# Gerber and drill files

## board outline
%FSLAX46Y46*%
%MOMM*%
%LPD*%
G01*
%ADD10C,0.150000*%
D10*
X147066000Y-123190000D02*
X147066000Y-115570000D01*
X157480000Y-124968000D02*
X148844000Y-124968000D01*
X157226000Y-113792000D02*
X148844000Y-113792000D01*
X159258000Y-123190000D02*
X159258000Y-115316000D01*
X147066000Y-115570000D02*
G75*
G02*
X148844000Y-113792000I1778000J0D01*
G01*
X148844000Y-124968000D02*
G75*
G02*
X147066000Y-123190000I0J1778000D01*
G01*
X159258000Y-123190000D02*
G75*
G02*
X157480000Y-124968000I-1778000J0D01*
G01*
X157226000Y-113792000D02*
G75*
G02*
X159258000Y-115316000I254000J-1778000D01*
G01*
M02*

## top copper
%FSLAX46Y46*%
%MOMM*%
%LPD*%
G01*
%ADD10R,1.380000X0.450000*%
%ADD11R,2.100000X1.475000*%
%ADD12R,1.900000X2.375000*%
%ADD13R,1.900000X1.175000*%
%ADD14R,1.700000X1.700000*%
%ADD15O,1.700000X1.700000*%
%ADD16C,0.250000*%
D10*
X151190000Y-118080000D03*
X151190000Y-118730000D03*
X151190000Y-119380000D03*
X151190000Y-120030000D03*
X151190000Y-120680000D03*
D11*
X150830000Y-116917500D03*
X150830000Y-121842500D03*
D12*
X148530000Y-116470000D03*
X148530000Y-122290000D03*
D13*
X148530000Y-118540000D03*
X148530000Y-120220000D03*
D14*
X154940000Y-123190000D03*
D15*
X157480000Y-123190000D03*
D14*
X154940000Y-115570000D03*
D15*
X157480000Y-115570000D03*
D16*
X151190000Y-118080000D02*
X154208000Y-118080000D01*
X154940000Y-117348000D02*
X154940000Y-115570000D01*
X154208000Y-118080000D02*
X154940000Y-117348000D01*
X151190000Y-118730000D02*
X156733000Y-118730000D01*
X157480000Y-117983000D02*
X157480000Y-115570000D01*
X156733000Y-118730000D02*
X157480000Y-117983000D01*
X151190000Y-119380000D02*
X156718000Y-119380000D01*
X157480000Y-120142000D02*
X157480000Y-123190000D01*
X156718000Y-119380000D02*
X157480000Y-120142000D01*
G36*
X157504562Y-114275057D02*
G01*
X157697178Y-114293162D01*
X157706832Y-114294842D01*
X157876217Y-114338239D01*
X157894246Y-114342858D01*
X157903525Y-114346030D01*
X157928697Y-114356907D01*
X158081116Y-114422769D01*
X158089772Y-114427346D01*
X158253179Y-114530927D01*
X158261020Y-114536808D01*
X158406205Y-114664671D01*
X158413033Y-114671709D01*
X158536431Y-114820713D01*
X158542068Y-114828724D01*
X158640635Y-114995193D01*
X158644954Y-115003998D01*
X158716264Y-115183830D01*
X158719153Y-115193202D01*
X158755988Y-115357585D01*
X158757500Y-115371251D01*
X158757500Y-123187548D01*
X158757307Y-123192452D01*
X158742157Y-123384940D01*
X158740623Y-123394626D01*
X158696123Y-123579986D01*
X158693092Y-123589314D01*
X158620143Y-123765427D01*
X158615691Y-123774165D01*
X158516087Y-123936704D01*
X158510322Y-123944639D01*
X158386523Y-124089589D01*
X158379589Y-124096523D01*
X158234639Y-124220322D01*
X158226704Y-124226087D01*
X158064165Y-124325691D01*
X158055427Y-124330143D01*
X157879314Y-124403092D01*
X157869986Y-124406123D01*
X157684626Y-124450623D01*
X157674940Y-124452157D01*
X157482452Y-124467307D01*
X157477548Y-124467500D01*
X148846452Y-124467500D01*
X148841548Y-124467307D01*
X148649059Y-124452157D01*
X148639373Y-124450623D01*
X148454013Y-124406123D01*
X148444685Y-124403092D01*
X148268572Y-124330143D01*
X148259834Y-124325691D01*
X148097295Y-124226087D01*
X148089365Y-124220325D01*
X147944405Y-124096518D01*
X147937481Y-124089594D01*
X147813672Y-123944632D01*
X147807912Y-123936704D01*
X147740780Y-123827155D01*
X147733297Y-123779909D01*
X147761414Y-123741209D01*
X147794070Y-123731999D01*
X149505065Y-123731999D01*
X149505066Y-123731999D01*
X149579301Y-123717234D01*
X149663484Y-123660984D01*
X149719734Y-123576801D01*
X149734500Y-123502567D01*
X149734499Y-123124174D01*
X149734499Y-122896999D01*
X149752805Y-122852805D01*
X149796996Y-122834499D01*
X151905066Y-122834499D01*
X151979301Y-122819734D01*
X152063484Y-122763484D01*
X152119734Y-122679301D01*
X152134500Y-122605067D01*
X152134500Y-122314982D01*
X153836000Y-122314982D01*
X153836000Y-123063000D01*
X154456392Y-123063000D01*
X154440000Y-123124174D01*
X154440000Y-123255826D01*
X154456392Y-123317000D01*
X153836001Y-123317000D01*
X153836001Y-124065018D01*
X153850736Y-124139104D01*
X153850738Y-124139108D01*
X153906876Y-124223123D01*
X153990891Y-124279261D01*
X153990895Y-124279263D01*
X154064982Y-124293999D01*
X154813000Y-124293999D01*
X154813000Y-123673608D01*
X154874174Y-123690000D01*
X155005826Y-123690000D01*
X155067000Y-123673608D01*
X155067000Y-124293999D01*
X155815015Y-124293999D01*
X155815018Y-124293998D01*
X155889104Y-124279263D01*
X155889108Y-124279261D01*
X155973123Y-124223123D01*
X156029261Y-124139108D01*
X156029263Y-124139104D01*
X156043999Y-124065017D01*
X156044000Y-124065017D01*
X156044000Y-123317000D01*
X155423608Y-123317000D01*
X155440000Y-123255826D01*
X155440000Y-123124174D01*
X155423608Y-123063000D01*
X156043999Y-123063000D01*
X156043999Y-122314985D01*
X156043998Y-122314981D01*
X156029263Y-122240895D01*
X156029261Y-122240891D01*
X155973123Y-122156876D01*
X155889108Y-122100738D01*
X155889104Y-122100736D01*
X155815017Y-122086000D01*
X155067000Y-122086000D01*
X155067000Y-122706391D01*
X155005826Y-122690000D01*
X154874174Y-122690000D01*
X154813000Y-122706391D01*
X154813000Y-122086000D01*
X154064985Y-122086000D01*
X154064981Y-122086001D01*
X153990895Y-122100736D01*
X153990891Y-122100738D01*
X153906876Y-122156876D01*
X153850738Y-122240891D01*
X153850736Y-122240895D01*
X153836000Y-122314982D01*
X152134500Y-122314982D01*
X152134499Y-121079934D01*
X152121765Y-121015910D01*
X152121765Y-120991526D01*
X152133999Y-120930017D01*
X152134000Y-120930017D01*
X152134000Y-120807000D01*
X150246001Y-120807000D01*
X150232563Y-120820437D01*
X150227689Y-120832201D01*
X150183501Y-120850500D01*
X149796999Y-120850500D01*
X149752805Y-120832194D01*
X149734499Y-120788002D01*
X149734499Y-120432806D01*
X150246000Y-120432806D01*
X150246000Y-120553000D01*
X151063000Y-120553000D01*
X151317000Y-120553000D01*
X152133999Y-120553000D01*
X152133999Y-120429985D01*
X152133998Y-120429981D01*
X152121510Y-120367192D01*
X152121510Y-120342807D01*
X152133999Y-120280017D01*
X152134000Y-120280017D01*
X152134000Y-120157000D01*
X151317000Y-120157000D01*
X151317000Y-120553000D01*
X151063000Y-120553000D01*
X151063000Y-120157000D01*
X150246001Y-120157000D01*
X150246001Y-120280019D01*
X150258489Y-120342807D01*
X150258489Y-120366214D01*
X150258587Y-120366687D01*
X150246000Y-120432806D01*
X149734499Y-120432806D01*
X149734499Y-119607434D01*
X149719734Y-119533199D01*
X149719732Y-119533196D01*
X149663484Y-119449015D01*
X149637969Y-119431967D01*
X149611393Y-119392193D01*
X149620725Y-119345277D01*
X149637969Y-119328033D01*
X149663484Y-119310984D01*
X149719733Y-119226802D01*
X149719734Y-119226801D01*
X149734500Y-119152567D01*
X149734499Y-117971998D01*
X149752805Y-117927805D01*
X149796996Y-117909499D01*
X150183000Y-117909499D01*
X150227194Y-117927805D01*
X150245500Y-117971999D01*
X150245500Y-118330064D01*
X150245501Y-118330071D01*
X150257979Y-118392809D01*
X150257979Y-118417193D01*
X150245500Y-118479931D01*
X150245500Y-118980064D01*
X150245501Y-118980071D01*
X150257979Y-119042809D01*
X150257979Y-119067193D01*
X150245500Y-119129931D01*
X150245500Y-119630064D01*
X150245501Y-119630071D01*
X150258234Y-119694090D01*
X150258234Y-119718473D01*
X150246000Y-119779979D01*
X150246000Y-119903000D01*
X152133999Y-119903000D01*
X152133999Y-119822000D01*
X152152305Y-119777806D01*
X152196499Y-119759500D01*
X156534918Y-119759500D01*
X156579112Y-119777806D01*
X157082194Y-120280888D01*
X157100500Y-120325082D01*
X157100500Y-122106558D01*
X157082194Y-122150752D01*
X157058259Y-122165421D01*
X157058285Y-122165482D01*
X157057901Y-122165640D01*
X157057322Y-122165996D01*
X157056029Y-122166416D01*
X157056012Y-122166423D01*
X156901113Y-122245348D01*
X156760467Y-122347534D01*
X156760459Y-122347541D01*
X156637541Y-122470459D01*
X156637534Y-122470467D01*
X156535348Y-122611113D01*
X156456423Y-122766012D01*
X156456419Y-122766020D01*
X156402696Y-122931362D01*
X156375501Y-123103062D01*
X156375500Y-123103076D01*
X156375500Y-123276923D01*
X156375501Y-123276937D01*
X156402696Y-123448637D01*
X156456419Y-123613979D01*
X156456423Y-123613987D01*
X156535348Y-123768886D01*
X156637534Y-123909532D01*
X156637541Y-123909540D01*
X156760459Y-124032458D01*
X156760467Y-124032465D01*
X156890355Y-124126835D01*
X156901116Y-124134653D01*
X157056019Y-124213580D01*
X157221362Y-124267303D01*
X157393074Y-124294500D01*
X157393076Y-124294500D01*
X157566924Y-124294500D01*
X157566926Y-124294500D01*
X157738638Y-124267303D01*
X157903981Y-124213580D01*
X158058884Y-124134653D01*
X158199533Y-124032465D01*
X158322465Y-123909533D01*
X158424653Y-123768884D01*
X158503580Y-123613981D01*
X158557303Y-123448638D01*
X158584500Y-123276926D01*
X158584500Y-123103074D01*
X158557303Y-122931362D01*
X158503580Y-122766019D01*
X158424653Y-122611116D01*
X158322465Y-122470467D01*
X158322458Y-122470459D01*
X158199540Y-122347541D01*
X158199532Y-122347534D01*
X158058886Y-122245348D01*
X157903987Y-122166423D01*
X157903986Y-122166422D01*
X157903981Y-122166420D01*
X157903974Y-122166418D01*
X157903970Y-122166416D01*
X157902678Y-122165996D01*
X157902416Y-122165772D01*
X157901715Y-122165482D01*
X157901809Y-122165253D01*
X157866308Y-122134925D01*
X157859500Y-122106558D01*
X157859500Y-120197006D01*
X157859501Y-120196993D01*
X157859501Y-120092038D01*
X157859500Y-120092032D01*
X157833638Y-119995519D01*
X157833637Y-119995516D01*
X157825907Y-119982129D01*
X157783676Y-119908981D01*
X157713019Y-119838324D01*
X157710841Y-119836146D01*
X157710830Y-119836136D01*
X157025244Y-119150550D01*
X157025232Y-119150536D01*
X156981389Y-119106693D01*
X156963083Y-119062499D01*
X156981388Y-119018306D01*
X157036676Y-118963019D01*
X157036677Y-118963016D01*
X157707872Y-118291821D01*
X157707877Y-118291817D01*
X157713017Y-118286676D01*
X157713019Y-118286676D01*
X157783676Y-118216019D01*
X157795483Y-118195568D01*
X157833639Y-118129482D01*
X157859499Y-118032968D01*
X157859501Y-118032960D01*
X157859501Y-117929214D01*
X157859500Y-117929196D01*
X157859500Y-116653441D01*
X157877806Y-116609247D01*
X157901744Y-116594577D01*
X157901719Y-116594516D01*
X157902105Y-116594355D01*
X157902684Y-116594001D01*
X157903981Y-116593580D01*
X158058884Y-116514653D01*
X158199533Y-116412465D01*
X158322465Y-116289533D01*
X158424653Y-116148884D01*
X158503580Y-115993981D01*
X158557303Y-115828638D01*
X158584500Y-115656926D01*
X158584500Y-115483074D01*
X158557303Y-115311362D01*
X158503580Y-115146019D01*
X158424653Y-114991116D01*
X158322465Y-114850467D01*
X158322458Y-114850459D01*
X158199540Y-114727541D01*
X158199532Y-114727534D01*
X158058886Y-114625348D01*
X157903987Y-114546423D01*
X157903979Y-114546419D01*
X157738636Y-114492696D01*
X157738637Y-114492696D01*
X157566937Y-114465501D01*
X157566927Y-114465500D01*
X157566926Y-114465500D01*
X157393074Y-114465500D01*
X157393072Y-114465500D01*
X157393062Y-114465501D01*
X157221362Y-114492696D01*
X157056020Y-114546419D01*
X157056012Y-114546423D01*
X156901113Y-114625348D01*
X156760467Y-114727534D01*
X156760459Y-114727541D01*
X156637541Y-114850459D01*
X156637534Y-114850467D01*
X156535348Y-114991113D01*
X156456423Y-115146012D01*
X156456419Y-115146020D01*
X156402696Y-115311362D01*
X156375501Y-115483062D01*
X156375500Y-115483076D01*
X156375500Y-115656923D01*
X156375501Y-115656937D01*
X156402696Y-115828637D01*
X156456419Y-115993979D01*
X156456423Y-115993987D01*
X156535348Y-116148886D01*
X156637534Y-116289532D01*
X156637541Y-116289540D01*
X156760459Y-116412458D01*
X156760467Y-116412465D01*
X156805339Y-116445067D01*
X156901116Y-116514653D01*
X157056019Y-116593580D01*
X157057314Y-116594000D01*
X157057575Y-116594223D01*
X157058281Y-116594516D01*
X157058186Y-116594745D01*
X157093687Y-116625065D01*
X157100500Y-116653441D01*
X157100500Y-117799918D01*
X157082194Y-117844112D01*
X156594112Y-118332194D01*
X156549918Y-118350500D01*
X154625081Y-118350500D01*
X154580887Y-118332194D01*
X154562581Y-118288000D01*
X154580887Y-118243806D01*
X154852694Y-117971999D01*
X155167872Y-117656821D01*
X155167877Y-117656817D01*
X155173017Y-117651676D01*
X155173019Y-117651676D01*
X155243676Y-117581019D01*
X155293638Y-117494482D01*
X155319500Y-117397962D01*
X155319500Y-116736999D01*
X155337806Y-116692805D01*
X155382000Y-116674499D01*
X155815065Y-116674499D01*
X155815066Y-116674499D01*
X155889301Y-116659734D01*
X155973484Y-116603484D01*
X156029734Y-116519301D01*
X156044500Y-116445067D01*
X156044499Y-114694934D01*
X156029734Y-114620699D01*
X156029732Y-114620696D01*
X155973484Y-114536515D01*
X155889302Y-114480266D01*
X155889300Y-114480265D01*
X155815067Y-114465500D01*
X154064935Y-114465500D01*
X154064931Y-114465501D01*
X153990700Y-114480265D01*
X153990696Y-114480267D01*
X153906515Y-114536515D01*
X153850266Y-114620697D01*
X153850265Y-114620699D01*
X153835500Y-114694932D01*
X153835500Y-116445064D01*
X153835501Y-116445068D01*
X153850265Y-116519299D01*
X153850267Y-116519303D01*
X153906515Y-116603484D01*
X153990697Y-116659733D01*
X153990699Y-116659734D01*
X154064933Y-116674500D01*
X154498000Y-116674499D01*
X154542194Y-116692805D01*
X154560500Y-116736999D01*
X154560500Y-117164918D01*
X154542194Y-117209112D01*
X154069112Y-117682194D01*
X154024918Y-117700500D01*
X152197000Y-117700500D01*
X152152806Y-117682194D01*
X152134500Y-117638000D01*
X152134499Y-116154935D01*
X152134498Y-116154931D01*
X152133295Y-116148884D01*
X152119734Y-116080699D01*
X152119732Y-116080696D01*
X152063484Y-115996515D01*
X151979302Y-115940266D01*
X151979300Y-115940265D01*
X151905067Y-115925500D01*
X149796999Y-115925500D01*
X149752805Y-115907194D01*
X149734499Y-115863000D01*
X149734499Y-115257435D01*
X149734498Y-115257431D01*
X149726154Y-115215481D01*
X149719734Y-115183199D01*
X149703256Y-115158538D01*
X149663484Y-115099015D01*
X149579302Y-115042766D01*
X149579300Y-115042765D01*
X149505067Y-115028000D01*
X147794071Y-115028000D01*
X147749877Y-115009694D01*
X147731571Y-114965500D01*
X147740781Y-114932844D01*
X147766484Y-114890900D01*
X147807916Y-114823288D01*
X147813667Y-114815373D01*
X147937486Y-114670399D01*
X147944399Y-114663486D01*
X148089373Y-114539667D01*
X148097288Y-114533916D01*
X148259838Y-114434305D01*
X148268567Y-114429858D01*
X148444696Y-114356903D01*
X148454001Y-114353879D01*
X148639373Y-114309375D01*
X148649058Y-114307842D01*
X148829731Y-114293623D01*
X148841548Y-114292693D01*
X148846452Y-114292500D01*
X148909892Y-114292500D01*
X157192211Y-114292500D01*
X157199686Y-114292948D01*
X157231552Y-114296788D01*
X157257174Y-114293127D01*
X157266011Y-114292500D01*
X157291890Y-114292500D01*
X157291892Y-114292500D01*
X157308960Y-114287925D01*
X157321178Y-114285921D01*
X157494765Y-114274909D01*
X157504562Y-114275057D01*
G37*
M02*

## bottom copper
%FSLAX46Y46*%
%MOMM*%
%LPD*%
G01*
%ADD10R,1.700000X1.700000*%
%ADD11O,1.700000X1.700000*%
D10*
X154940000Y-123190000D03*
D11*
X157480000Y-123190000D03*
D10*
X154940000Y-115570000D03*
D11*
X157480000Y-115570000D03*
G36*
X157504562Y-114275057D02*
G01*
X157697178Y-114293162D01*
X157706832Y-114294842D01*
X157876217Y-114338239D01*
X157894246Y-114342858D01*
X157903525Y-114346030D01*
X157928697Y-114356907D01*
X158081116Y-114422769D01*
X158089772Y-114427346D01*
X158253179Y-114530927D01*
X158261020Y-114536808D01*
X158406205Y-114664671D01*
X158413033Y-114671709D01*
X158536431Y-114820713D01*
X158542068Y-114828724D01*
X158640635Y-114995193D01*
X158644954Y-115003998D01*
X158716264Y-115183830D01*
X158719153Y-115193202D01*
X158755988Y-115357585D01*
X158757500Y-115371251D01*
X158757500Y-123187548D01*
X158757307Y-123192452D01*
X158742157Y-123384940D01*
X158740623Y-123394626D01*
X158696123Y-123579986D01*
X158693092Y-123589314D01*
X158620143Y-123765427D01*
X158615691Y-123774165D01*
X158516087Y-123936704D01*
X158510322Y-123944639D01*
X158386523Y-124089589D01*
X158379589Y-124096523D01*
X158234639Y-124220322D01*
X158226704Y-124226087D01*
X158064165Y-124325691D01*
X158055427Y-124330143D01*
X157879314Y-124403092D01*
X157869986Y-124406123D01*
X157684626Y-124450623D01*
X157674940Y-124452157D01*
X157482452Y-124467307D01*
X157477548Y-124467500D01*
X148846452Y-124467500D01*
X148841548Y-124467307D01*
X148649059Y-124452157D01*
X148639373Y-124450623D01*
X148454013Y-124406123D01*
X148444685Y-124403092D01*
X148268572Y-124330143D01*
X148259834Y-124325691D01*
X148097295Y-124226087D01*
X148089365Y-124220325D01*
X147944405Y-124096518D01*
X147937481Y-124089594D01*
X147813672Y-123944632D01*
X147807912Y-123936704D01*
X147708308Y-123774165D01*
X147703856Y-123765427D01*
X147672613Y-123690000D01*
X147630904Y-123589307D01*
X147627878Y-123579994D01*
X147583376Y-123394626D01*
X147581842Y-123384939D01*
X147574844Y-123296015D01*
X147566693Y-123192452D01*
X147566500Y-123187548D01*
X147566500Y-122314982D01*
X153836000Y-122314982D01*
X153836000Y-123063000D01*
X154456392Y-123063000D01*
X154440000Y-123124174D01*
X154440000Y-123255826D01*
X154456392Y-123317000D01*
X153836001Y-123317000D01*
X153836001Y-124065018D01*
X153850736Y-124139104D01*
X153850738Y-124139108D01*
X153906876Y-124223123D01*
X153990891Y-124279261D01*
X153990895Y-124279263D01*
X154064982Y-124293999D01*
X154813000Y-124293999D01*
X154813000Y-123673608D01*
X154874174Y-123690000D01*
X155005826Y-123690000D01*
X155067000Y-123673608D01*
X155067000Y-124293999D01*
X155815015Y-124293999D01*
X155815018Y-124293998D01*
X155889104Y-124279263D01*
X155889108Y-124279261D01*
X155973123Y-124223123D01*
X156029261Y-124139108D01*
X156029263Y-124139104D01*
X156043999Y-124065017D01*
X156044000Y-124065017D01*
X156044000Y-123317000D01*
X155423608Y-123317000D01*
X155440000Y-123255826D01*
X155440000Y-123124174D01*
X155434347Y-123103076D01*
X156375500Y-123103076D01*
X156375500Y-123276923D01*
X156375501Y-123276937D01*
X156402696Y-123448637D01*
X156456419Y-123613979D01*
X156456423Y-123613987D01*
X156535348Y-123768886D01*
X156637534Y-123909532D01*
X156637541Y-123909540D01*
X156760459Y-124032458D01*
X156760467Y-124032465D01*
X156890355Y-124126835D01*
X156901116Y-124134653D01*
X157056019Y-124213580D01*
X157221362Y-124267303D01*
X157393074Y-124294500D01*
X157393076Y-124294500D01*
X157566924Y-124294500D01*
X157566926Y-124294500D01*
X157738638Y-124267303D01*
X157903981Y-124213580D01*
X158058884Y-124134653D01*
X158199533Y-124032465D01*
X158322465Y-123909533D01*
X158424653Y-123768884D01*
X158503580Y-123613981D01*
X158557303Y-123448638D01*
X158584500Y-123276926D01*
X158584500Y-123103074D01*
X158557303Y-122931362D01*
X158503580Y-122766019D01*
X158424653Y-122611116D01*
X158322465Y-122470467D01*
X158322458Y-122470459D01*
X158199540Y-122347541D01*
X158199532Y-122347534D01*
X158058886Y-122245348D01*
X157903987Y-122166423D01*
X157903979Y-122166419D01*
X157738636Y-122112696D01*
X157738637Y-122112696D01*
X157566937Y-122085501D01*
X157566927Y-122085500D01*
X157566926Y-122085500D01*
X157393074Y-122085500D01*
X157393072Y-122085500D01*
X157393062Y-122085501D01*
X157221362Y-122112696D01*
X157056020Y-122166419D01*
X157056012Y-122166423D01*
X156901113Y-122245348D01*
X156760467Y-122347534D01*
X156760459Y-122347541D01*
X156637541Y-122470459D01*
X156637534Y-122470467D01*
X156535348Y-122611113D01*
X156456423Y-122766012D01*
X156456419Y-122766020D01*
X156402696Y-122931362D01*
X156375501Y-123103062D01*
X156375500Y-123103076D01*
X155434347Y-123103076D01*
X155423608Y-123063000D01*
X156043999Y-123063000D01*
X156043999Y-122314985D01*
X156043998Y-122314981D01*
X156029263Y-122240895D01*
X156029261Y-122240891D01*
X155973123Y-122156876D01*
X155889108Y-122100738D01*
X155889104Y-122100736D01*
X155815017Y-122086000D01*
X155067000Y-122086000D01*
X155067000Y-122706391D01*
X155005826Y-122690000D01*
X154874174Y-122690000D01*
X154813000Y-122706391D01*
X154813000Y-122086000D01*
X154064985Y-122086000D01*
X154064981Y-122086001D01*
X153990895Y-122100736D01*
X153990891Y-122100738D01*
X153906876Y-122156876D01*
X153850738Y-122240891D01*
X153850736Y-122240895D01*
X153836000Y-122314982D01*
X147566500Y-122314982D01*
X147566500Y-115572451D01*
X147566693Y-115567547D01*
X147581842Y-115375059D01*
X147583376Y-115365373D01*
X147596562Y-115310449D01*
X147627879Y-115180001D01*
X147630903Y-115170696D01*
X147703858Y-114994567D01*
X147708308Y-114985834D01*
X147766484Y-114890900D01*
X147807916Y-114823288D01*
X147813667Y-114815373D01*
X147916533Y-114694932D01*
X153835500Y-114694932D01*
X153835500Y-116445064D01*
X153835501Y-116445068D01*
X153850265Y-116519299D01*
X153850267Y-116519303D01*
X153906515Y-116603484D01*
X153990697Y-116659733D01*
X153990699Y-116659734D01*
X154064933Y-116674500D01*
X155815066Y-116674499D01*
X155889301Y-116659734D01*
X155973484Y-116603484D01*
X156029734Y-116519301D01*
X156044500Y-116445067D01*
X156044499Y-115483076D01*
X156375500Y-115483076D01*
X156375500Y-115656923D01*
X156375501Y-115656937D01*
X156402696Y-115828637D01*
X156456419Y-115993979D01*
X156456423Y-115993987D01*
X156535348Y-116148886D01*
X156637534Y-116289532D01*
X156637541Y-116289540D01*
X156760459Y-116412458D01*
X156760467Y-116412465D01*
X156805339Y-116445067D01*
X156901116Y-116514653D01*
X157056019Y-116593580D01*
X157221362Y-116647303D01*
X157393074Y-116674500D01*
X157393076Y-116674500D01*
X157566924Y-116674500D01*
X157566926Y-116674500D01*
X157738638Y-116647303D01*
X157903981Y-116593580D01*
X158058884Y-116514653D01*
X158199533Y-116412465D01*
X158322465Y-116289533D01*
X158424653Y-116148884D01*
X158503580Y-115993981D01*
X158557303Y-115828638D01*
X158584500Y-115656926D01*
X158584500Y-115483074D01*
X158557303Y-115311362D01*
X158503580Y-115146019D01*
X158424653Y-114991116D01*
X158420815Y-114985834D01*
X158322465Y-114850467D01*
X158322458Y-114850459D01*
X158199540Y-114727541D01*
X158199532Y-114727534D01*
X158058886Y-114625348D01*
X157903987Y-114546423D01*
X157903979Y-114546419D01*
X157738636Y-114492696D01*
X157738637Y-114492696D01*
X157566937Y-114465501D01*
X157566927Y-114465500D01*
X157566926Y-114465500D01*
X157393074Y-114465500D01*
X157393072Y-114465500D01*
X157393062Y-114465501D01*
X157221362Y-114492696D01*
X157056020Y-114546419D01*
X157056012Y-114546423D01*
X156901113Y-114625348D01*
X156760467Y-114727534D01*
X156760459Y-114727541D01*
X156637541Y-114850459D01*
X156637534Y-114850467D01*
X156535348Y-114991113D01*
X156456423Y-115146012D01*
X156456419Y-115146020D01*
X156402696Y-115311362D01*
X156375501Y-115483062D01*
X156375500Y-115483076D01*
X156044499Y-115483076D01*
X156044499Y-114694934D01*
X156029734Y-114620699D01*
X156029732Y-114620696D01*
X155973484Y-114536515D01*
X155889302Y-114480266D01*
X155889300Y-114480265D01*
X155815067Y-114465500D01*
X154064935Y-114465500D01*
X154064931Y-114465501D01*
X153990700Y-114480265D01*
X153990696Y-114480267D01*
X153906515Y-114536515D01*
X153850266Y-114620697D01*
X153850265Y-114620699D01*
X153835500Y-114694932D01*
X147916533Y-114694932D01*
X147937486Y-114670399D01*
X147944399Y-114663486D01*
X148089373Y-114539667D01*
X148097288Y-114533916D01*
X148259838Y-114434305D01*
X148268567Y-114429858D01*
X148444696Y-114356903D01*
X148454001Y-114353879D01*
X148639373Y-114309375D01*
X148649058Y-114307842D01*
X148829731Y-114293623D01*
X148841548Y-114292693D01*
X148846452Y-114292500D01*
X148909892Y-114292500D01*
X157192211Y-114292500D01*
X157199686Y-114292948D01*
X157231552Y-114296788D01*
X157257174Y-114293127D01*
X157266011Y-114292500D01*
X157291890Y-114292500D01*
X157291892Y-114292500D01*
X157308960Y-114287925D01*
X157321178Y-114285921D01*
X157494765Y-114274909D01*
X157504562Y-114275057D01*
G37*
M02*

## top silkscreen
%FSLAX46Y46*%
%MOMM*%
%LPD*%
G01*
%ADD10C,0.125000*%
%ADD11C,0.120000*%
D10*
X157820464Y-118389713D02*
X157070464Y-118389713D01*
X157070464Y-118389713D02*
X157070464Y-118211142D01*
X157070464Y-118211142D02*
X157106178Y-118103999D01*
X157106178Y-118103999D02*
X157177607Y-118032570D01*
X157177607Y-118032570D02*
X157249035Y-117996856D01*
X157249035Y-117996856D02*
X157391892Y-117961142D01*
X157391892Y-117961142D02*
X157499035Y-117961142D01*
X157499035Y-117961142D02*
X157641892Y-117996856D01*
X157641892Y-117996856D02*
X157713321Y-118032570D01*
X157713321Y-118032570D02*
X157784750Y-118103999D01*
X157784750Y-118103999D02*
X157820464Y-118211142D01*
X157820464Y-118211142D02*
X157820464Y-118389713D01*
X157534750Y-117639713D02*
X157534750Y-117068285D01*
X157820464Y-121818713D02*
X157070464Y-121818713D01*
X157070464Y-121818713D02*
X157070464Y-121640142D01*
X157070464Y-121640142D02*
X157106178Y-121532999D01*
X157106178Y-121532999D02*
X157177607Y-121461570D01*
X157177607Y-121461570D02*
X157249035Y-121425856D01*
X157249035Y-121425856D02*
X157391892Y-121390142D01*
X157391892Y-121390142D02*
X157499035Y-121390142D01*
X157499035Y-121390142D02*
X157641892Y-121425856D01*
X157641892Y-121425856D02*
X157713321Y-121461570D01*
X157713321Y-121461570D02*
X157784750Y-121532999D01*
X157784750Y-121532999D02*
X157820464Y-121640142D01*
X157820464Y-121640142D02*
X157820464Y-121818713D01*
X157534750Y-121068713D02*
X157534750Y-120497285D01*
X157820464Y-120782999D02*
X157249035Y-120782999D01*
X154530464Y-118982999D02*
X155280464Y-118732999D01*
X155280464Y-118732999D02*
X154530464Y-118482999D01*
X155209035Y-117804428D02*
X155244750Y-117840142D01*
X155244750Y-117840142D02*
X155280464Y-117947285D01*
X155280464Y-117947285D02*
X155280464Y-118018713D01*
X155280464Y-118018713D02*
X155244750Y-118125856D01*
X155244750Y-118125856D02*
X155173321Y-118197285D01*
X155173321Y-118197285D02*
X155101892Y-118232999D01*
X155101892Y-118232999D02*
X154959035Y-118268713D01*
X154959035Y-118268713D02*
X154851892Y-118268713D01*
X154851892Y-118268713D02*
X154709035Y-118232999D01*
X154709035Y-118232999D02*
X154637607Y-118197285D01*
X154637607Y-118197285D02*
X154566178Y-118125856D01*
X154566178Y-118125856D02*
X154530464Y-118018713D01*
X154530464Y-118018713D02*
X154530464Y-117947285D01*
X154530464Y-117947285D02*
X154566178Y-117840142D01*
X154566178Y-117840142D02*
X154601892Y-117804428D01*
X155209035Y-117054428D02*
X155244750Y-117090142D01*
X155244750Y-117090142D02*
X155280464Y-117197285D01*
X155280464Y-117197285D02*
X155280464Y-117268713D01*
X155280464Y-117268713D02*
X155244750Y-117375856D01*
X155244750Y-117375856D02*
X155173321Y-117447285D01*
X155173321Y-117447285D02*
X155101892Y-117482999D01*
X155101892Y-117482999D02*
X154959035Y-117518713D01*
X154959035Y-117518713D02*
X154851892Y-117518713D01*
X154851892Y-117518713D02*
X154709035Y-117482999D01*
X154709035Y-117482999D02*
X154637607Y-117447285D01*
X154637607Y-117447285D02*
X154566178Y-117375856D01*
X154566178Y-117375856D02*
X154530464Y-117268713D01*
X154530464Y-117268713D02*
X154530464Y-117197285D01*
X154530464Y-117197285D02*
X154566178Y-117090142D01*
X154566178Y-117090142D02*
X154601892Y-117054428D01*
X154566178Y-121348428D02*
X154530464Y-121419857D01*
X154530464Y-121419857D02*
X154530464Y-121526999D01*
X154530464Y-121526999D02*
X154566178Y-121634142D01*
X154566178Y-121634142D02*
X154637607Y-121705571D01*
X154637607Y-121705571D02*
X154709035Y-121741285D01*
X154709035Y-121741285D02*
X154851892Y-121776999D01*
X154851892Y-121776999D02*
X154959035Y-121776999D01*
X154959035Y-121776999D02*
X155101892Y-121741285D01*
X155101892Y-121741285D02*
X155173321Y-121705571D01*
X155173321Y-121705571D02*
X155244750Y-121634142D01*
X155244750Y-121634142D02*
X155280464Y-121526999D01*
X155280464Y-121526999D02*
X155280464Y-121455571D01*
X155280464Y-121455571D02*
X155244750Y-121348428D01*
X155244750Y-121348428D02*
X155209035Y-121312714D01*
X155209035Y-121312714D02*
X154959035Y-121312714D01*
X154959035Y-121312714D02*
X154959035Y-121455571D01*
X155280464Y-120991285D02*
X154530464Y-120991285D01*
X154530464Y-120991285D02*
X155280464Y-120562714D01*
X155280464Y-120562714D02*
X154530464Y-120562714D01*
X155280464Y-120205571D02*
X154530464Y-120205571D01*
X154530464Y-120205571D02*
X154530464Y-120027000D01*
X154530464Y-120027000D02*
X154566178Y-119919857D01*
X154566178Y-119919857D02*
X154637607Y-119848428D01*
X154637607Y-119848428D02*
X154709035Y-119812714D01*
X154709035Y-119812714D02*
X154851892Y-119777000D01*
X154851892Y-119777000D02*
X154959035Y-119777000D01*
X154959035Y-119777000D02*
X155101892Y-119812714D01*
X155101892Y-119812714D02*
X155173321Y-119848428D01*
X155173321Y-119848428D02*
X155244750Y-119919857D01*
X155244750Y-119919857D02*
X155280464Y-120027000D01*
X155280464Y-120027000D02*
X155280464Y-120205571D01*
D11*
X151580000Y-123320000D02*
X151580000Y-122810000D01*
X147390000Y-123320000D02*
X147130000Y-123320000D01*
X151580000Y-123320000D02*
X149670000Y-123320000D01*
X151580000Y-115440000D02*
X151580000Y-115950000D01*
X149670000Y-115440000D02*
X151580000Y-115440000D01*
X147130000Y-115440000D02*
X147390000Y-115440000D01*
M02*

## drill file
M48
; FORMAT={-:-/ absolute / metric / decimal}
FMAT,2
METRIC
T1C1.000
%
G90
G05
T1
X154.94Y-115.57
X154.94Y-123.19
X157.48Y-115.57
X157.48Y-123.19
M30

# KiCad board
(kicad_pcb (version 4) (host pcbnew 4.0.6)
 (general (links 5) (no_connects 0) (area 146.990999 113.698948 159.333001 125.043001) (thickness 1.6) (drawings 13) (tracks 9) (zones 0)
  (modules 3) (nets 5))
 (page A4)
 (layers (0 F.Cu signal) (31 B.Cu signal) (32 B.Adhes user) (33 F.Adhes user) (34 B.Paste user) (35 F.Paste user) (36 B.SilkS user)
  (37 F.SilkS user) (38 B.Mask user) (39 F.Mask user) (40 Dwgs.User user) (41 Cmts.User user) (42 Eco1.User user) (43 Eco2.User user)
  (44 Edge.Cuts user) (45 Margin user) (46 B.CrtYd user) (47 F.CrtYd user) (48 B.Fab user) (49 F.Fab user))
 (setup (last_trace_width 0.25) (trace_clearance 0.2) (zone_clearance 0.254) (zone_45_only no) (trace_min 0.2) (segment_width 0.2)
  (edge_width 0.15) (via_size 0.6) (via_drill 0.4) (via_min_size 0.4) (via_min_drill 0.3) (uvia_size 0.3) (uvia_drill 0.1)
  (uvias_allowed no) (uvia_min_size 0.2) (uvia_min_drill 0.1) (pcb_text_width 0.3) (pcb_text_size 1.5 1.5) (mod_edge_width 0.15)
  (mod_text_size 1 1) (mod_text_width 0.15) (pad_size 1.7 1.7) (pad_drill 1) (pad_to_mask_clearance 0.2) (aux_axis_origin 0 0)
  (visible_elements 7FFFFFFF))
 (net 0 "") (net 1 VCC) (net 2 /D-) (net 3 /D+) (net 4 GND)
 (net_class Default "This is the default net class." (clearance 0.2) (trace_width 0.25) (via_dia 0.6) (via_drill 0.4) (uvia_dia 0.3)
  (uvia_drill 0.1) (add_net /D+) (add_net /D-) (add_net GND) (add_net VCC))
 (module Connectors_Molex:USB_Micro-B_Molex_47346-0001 (layer F.Cu) (at 149.86 119.38)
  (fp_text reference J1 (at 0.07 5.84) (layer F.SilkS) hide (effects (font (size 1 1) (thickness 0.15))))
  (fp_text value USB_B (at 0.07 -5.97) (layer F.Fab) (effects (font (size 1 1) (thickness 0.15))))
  (fp_line (start 1.72 3.94) (end 1.72 3.43) (layer F.SilkS) (width 0.12))
  (fp_line (start -2.47 3.94) (end -2.73 3.94) (layer F.SilkS) (width 0.12))
  (fp_line (start 1.72 3.94) (end -0.19 3.94) (layer F.SilkS) (width 0.12))
  (fp_line (start 1.72 -3.94) (end 1.72 -3.43) (layer F.SilkS) (width 0.12))
  (fp_line (start -0.19 -3.94) (end 1.72 -3.94) (layer F.SilkS) (width 0.12))
  (fp_line (start -2.73 -3.94) (end -2.47 -3.94) (layer F.SilkS) (width 0.12))
  (pad 1 smd rect (at 1.33 -1.3) (size 1.38 0.45) (layers F.Cu F.Paste F.Mask) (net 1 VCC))
  (pad 2 smd rect (at 1.33 -0.65) (size 1.38 0.45) (layers F.Cu F.Paste F.Mask) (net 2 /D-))
  (pad 3 smd rect (at 1.33 0) (size 1.38 0.45) (layers F.Cu F.Paste F.Mask) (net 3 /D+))
  (pad 4 smd rect (at 1.33 0.65) (size 1.38 0.45) (layers F.Cu F.Paste F.Mask) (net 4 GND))
  (pad 5 smd rect (at 1.33 1.3) (size 1.38 0.45) (layers F.Cu F.Paste F.Mask) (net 4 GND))
  (pad 6 smd rect (at 0.97 -2.4625) (size 2.1 1.475) (layers F.Cu F.Paste F.Mask))
  (pad 6 smd rect (at 0.97 2.4625) (size 2.1 1.475) (layers F.Cu F.Paste F.Mask))
  (pad 6 smd rect (at -1.33 -2.91) (size 1.9 2.375) (layers F.Cu F.Paste F.Mask))
  (pad 6 smd rect (at -1.33 2.91) (size 1.9 2.375) (layers F.Cu F.Paste F.Mask))
  (pad 6 smd rect (at -1.33 -0.84) (size 1.9 1.175) (layers F.Cu F.Paste F.Mask))
  (pad 6 smd rect (at -1.33 0.84) (size 1.9 1.175) (layers F.Cu F.Paste F.Mask)))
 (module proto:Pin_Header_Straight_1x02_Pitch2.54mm (layer F.Cu) (at 154.94 123.19 90)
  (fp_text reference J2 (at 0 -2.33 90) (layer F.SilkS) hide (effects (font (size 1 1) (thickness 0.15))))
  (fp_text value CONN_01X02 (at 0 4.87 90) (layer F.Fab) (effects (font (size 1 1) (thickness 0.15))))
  (pad 1 thru_hole rect (at 0 0 90) (size 1.7 1.7) (drill 1) (layers *.Cu *.Mask) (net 4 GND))
  (pad 2 thru_hole oval (at 0 2.54 90) (size 1.7 1.7) (drill 1) (layers *.Cu *.Mask) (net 3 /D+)))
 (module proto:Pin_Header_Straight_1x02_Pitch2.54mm (layer F.Cu) (at 154.94 115.57 90)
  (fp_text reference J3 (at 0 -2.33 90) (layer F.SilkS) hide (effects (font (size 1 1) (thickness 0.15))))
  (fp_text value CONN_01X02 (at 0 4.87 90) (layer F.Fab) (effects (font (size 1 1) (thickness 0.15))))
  (pad 1 thru_hole rect (at 0 0 90) (size 1.7 1.7) (drill 1) (layers *.Cu *.Mask) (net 1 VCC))
  (pad 2 thru_hole oval (at 0 2.54 90) (size 1.7 1.7) (drill 1) (layers *.Cu *.Mask) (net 2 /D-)))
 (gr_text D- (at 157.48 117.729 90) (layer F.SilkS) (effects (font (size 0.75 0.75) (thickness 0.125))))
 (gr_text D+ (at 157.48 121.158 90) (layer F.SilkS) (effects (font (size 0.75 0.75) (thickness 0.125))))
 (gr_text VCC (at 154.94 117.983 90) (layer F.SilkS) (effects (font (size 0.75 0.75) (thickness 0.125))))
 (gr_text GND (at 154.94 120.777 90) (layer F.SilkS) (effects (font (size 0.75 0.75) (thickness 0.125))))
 (gr_line (start 147.066 123.19) (end 147.066 115.57) (angle 90) (layer Edge.Cuts) (width 0.15))
 (gr_line (start 157.48 124.968) (end 148.844 124.968) (angle 90) (layer Edge.Cuts) (width 0.15))
 (gr_line (start 157.226 113.792) (end 148.844 113.792) (angle 90) (layer Edge.Cuts) (width 0.15))
 (gr_line (start 159.258 123.19) (end 159.258 115.316) (angle 90) (layer Edge.Cuts) (width 0.15))
 (gr_arc (start 148.844 115.57) (end 147.066 115.57) (angle 90) (layer Edge.Cuts) (width 0.15))
 (gr_arc (start 148.844 123.19) (end 148.844 124.968) (angle 90) (layer Edge.Cuts) (width 0.15))
 (gr_arc (start 157.48 123.19) (end 159.258 123.19) (angle 90) (layer Edge.Cuts) (width 0.15))
 (gr_arc (start 157.48 115.57) (end 157.226 113.792) (angle 90) (layer Edge.Cuts) (width 0.15))
 (segment (start 151.19 118.08) (end 154.208 118.08) (width 0.25) (layer F.Cu) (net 1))
 (segment (start 154.94 117.348) (end 154.94 115.57) (width 0.25) (layer F.Cu) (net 1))
 (segment (start 154.208 118.08) (end 154.94 117.348) (width 0.25) (layer F.Cu) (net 1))
 (segment (start 151.19 118.73) (end 156.733 118.73) (width 0.25) (layer F.Cu) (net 2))
 (segment (start 157.48 117.983) (end 157.48 115.57) (width 0.25) (layer F.Cu) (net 2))
 (segment (start 156.733 118.73) (end 157.48 117.983) (width 0.25) (layer F.Cu) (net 2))
 (segment (start 151.19 119.38) (end 156.718 119.38) (width 0.25) (layer F.Cu) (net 3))
 (segment (start 157.48 120.142) (end 157.48 123.19) (width 0.25) (layer F.Cu) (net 3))
 (segment (start 156.718 119.38) (end 157.48 120.142) (width 0.25) (layer F.Cu) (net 3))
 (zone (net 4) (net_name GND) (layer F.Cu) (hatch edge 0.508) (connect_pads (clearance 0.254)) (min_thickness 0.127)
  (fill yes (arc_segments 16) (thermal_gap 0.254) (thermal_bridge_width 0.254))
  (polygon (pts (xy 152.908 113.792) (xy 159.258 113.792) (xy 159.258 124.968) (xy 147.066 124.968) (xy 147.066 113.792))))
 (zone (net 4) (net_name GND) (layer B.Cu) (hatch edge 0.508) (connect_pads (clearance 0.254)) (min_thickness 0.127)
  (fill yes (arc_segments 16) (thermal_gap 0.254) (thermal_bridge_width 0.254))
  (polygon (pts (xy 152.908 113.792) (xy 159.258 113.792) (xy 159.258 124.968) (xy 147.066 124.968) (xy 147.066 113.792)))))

